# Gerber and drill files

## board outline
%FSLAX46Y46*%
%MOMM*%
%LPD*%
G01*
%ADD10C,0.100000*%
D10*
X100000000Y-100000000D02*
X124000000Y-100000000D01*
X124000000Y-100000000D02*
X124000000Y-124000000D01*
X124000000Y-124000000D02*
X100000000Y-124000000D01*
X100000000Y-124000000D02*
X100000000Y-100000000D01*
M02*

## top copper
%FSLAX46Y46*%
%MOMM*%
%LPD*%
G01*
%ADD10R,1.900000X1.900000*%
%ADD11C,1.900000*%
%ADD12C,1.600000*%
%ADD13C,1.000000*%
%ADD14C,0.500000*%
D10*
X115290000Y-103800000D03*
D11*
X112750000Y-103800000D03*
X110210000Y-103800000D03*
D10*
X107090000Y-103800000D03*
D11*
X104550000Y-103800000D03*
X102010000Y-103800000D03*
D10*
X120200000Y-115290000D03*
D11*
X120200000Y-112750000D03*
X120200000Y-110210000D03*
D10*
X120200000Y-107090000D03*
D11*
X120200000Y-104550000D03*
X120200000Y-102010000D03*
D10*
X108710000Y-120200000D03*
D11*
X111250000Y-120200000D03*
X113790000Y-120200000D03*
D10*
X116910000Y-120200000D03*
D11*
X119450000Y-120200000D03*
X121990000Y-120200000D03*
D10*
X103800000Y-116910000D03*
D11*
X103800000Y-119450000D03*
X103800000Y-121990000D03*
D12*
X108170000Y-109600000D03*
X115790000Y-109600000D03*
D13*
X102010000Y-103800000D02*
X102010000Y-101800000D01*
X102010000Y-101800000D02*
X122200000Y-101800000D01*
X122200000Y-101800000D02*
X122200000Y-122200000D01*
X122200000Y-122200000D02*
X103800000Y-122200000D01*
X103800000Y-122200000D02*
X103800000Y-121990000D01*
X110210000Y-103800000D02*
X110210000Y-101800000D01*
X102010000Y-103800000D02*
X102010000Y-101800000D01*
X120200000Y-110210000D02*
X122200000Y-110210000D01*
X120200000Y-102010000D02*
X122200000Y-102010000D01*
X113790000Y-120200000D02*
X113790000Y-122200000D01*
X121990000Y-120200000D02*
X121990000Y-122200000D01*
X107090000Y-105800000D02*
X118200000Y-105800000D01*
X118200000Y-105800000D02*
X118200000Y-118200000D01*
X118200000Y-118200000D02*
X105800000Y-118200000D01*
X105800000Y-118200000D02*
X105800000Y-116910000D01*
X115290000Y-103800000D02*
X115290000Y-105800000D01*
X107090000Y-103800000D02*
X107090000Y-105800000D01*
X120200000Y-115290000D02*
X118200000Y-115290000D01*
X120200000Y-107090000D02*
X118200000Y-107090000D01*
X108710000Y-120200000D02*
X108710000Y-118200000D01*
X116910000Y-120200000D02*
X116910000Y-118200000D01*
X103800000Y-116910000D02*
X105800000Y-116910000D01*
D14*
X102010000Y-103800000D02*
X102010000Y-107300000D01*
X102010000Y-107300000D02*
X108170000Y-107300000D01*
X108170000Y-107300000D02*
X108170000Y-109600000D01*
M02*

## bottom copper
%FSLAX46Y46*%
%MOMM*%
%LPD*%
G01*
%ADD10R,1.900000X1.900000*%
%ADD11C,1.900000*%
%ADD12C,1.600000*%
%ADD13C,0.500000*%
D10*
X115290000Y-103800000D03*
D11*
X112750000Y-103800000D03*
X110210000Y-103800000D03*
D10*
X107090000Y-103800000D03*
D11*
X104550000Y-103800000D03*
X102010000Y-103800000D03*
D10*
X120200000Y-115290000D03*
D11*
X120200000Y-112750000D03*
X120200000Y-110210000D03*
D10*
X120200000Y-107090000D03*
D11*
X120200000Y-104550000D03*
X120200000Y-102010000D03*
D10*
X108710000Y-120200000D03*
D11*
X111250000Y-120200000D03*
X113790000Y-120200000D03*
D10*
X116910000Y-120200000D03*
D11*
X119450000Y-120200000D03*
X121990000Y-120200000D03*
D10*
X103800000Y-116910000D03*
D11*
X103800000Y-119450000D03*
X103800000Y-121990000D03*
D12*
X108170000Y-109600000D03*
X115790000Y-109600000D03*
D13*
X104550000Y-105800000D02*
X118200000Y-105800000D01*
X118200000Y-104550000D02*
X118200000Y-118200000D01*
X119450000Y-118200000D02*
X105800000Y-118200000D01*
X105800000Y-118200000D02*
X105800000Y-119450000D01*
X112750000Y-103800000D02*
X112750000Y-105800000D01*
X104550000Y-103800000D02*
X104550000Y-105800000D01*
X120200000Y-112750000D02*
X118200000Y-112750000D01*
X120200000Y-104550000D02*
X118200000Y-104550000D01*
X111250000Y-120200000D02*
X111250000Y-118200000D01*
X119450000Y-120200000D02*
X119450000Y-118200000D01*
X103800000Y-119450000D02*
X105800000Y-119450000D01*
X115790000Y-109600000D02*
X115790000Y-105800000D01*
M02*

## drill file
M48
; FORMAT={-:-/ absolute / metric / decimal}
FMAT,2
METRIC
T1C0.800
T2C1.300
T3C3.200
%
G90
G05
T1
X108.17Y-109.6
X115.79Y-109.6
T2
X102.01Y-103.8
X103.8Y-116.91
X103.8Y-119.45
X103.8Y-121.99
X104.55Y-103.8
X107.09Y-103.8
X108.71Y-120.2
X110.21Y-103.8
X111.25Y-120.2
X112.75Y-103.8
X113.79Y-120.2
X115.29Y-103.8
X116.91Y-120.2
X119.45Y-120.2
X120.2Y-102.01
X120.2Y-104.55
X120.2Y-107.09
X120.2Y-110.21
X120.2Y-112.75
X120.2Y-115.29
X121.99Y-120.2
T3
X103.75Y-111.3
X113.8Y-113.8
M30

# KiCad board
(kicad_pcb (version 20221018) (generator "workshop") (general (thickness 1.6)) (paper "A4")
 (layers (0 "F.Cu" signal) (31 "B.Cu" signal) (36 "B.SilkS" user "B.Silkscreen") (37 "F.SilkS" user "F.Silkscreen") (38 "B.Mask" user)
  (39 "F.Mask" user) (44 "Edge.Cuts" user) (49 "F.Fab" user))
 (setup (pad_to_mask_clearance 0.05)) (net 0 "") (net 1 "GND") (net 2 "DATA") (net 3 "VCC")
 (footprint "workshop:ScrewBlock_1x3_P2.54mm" (layer "F.Cu") (at 115.290 103.800 180)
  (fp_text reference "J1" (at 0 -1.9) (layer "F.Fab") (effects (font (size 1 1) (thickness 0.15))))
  (pad "1" thru_hole rect (at 0.000 0 180) (size 1.9 1.9) (drill 1.3) (layers "*.Cu" "*.Mask") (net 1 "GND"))
  (pad "2" thru_hole circle (at 2.540 0 180) (size 1.9 1.9) (drill 1.3) (layers "*.Cu" "*.Mask") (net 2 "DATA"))
  (pad "3" thru_hole circle (at 5.080 0 180) (size 1.9 1.9) (drill 1.3) (layers "*.Cu" "*.Mask") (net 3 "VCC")))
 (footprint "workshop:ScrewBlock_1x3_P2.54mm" (layer "F.Cu") (at 107.090 103.800 180)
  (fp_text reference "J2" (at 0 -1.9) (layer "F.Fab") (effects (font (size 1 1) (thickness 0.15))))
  (pad "1" thru_hole rect (at 0.000 0 180) (size 1.9 1.9) (drill 1.3) (layers "*.Cu" "*.Mask") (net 1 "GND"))
  (pad "2" thru_hole circle (at 2.540 0 180) (size 1.9 1.9) (drill 1.3) (layers "*.Cu" "*.Mask") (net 2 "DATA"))
  (pad "3" thru_hole circle (at 5.080 0 180) (size 1.9 1.9) (drill 1.3) (layers "*.Cu" "*.Mask") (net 3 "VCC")))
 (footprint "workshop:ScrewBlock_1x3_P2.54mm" (layer "F.Cu") (at 120.200 115.290 90)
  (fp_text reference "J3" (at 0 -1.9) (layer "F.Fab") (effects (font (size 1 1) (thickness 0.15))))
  (pad "1" thru_hole rect (at 0.000 0 90) (size 1.9 1.9) (drill 1.3) (layers "*.Cu" "*.Mask") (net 1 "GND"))
  (pad "2" thru_hole circle (at 2.540 0 90) (size 1.9 1.9) (drill 1.3) (layers "*.Cu" "*.Mask") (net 2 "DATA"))
  (pad "3" thru_hole circle (at 5.080 0 90) (size 1.9 1.9) (drill 1.3) (layers "*.Cu" "*.Mask") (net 3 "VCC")))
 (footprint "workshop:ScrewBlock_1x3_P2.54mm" (layer "F.Cu") (at 120.200 107.090 90)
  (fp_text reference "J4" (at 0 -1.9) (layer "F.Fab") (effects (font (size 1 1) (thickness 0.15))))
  (pad "1" thru_hole rect (at 0.000 0 90) (size 1.9 1.9) (drill 1.3) (layers "*.Cu" "*.Mask") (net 1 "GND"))
  (pad "2" thru_hole circle (at 2.540 0 90) (size 1.9 1.9) (drill 1.3) (layers "*.Cu" "*.Mask") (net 2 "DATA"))
  (pad "3" thru_hole circle (at 5.080 0 90) (size 1.9 1.9) (drill 1.3) (layers "*.Cu" "*.Mask") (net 3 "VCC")))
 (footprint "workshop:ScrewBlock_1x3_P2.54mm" (layer "F.Cu") (at 108.710 120.200 0)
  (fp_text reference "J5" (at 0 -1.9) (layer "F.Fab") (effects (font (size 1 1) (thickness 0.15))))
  (pad "1" thru_hole rect (at 0.000 0 0) (size 1.9 1.9) (drill 1.3) (layers "*.Cu" "*.Mask") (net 1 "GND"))
  (pad "2" thru_hole circle (at 2.540 0 0) (size 1.9 1.9) (drill 1.3) (layers "*.Cu" "*.Mask") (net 2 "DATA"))
  (pad "3" thru_hole circle (at 5.080 0 0) (size 1.9 1.9) (drill 1.3) (layers "*.Cu" "*.Mask") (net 3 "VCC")))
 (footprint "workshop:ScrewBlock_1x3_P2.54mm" (layer "F.Cu") (at 116.910 120.200 0)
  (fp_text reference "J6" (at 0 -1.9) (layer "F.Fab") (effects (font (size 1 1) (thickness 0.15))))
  (pad "1" thru_hole rect (at 0.000 0 0) (size 1.9 1.9) (drill 1.3) (layers "*.Cu" "*.Mask") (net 1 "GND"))
  (pad "2" thru_hole circle (at 2.540 0 0) (size 1.9 1.9) (drill 1.3) (layers "*.Cu" "*.Mask") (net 2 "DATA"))
  (pad "3" thru_hole circle (at 5.080 0 0) (size 1.9 1.9) (drill 1.3) (layers "*.Cu" "*.Mask") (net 3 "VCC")))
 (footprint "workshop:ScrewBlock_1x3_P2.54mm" (layer "F.Cu") (at 103.800 116.910 270)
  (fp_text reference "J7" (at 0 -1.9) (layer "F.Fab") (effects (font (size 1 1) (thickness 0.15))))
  (pad "1" thru_hole rect (at 0.000 0 270) (size 1.9 1.9) (drill 1.3) (layers "*.Cu" "*.Mask") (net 1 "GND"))
  (pad "2" thru_hole circle (at 2.540 0 270) (size 1.9 1.9) (drill 1.3) (layers "*.Cu" "*.Mask") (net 2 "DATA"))
  (pad "3" thru_hole circle (at 5.080 0 270) (size 1.9 1.9) (drill 1.3) (layers "*.Cu" "*.Mask") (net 3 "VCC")))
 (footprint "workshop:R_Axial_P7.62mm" (layer "F.Cu") (at 108.170 109.600)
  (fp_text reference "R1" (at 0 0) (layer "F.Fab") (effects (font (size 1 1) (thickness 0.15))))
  (pad "1" thru_hole circle (at 0.000 0.000) (size 1.6 1.6) (drill 0.8) (layers "*.Cu" "*.Mask") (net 3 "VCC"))
  (pad "2" thru_hole circle (at 7.620 0.000) (size 1.6 1.6) (drill 0.8) (layers "*.Cu" "*.Mask") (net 2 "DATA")))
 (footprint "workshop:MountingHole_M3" (layer "F.Cu") (at 103.750 111.300)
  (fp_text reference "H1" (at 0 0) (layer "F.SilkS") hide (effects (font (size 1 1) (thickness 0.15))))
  (pad "" np_thru_hole circle (at 0 0) (size 3.2 3.2) (drill 3.2) (layers "*.Cu" "*.Mask")))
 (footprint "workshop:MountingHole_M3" (layer "F.Cu") (at 113.800 113.800)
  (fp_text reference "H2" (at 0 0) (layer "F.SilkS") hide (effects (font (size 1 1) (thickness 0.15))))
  (pad "" np_thru_hole circle (at 0 0) (size 3.2 3.2) (drill 3.2) (layers "*.Cu" "*.Mask")))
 (segment (start 102.010 103.800) (end 102.010 101.800) (width 1.0) (layer "F.Cu") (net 3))
 (segment (start 102.010 101.800) (end 122.200 101.800) (width 1.0) (layer "F.Cu") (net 3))
 (segment (start 122.200 101.800) (end 122.200 122.200) (width 1.0) (layer "F.Cu") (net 3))
 (segment (start 122.200 122.200) (end 103.800 122.200) (width 1.0) (layer "F.Cu") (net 3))
 (segment (start 103.800 122.200) (end 103.800 121.990) (width 1.0) (layer "F.Cu") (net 3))
 (segment (start 110.210 103.800) (end 110.210 101.800) (width 1.0) (layer "F.Cu") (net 3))
 (segment (start 102.010 103.800) (end 102.010 101.800) (width 1.0) (layer "F.Cu") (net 3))
 (segment (start 120.200 110.210) (end 122.200 110.210) (width 1.0) (layer "F.Cu") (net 3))
 (segment (start 120.200 102.010) (end 122.200 102.010) (width 1.0) (layer "F.Cu") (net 3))
 (segment (start 113.790 120.200) (end 113.790 122.200) (width 1.0) (layer "F.Cu") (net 3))
 (segment (start 121.990 120.200) (end 121.990 122.200) (width 1.0) (layer "F.Cu") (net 3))
 (segment (start 107.090 105.800) (end 118.200 105.800) (width 1.0) (layer "F.Cu") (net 1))
 (segment (start 118.200 105.800) (end 118.200 118.200) (width 1.0) (layer "F.Cu") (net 1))
 (segment (start 118.200 118.200) (end 105.800 118.200) (width 1.0) (layer "F.Cu") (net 1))
 (segment (start 105.800 118.200) (end 105.800 116.910) (width 1.0) (layer "F.Cu") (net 1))
 (segment (start 115.290 103.800) (end 115.290 105.800) (width 1.0) (layer "F.Cu") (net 1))
 (segment (start 107.090 103.800) (end 107.090 105.800) (width 1.0) (layer "F.Cu") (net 1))
 (segment (start 120.200 115.290) (end 118.200 115.290) (width 1.0) (layer "F.Cu") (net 1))
 (segment (start 120.200 107.090) (end 118.200 107.090) (width 1.0) (layer "F.Cu") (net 1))
 (segment (start 108.710 120.200) (end 108.710 118.200) (width 1.0) (layer "F.Cu") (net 1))
 (segment (start 116.910 120.200) (end 116.910 118.200) (width 1.0) (layer "F.Cu") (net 1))
 (segment (start 103.800 116.910) (end 105.800 116.910) (width 1.0) (layer "F.Cu") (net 1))
 (segment (start 104.550 105.800) (end 118.200 105.800) (width 0.5) (layer "B.Cu") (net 2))
 (segment (start 118.200 104.550) (end 118.200 118.200) (width 0.5) (layer "B.Cu") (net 2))
 (segment (start 119.450 118.200) (end 105.800 118.200) (width 0.5) (layer "B.Cu") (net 2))
 (segment (start 105.800 118.200) (end 105.800 119.450) (width 0.5) (layer "B.Cu") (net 2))
 (segment (start 112.750 103.800) (end 112.750 105.800) (width 0.5) (layer "B.Cu") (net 2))
 (segment (start 104.550 103.800) (end 104.550 105.800) (width 0.5) (layer "B.Cu") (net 2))
 (segment (start 120.200 112.750) (end 118.200 112.750) (width 0.5) (layer "B.Cu") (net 2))
 (segment (start 120.200 104.550) (end 118.200 104.550) (width 0.5) (layer "B.Cu") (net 2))
 (segment (start 111.250 120.200) (end 111.250 118.200) (width 0.5) (layer "B.Cu") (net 2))
 (segment (start 119.450 120.200) (end 119.450 118.200) (width 0.5) (layer "B.Cu") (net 2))
 (segment (start 103.800 119.450) (end 105.800 119.450) (width 0.5) (layer "B.Cu") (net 2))
 (segment (start 102.010 103.800) (end 102.010 107.300) (width 0.5) (layer "F.Cu") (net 3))
 (segment (start 102.010 107.300) (end 108.170 107.300) (width 0.5) (layer "F.Cu") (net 3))
 (segment (start 108.170 107.300) (end 108.170 109.600) (width 0.5) (layer "F.Cu") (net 3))
 (segment (start 115.790 109.600) (end 115.790 105.800) (width 0.5) (layer "B.Cu") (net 2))
 (gr_line (start 100.000 100.000) (end 124.000 100.000) (layer "Edge.Cuts") (width 0.1))
 (gr_line (start 124.000 100.000) (end 124.000 124.000) (layer "Edge.Cuts") (width 0.1))
 (gr_line (start 124.000 124.000) (end 100.000 124.000) (layer "Edge.Cuts") (width 0.1))
 (gr_line (start 100.000 124.000) (end 100.000 100.000) (layer "Edge.Cuts") (width 0.1)))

